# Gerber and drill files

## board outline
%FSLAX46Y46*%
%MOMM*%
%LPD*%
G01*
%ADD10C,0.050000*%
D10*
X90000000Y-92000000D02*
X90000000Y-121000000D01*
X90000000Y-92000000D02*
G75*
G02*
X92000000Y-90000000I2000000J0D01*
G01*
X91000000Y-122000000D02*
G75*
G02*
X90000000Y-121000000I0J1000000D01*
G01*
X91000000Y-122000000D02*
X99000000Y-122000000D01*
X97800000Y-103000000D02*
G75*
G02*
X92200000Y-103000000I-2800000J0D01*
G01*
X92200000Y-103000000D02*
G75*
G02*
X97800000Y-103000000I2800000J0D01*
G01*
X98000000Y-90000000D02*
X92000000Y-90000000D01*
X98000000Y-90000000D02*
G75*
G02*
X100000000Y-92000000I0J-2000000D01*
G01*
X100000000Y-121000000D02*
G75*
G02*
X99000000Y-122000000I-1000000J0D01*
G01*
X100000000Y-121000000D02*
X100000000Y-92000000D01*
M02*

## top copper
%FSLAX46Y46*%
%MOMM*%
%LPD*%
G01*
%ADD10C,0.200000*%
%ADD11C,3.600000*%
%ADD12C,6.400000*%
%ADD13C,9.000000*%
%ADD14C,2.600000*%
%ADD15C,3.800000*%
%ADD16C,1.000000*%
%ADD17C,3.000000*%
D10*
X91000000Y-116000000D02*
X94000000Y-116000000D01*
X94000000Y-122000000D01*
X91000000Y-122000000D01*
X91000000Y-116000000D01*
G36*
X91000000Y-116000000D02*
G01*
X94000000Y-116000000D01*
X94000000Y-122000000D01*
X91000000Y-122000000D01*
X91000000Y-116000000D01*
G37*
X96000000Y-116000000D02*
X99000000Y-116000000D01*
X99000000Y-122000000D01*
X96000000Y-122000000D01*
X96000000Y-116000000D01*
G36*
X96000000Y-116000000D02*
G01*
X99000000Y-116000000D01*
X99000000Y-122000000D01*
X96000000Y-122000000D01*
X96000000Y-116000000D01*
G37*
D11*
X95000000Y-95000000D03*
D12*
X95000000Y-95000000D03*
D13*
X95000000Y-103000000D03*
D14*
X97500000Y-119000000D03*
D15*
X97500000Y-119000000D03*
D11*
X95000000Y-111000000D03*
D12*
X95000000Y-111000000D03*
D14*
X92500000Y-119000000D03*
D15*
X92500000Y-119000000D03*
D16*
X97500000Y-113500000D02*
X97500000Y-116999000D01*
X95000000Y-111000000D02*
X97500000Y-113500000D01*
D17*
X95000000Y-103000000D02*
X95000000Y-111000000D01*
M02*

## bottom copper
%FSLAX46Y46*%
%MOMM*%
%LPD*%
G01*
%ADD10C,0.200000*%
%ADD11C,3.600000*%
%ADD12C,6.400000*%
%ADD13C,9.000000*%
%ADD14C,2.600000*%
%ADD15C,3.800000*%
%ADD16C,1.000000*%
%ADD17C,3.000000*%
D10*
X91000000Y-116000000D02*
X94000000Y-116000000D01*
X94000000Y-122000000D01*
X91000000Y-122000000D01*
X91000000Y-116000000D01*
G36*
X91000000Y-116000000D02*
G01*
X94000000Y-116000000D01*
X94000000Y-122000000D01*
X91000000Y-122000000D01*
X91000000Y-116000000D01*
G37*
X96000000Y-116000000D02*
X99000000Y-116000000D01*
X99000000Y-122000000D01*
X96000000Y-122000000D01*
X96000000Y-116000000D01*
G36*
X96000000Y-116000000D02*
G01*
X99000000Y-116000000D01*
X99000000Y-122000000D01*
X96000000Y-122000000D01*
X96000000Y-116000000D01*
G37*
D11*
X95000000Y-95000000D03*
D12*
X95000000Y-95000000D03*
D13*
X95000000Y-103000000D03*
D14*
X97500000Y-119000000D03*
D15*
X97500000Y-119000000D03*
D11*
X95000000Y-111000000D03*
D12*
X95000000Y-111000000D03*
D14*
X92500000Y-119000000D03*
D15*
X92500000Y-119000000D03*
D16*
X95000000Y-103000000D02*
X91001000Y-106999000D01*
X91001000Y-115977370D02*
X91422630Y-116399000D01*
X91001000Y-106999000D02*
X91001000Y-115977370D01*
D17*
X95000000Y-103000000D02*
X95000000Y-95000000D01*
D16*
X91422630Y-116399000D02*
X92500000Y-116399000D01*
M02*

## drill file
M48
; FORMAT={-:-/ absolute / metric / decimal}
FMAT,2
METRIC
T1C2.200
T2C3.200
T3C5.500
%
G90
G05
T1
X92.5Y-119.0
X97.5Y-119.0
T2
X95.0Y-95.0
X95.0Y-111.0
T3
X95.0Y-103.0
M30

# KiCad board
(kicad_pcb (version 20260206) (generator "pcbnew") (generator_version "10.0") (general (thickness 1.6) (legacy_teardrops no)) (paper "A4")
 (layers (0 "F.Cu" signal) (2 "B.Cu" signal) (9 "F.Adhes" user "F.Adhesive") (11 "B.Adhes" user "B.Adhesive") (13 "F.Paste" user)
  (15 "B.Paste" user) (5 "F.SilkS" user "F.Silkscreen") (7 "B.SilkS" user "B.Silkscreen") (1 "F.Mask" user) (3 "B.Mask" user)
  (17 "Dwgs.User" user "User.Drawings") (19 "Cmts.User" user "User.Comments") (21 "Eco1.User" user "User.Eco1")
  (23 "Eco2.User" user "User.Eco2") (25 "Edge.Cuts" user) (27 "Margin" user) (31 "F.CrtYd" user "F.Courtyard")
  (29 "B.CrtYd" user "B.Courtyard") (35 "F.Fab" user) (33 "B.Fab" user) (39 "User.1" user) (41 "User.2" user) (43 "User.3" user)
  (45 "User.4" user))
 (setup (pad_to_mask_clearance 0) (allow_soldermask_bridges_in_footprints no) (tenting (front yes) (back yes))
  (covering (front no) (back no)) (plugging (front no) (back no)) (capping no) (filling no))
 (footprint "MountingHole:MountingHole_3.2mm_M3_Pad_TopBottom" (layer "F.Cu") (at 95 95)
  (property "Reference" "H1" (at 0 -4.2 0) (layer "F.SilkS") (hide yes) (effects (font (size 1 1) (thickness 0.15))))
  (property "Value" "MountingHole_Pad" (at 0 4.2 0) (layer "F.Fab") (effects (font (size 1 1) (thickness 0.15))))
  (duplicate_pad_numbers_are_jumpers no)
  (pad "1" thru_hole circle (at 0 0) (size 3.6 3.6) (drill 3.2) (layers "*.Cu" "*.Mask") (remove_unused_layers no)
   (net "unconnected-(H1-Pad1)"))
  (pad "1" connect circle (at 0 0) (size 6.4 6.4) (layers "F.Cu" "F.Mask") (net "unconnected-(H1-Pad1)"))
  (pad "1" connect circle (at 0 0) (size 6.4 6.4) (layers "B.Cu" "B.Mask") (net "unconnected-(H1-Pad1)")))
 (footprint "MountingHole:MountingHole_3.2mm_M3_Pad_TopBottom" (layer "F.Cu") (at 95 103)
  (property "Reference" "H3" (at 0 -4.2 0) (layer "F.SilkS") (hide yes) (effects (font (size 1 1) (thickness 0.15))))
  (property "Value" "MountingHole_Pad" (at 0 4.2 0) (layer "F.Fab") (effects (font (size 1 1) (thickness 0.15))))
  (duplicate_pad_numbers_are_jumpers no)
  (pad "" np_thru_hole circle (at 0 0) (size 5.5 5.5) (drill 5.5) (layers "*.Cu" "*.Mask"))
  (pad "1" connect circle (at 0 0) (size 9 9) (layers "F.Cu" "F.Mask") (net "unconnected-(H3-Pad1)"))
  (pad "e" connect circle (at 0 0) (size 9 9) (layers "B.Cu" "B.Mask")))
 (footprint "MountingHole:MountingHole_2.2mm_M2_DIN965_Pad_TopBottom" (layer "F.Cu") (at 97.5 119)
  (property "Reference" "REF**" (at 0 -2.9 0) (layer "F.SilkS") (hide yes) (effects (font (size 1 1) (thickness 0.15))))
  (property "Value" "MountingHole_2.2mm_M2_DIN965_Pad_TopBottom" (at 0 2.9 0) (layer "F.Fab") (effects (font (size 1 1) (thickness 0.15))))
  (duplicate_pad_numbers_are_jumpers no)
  (pad "1" thru_hole circle (at 0 0) (size 2.6 2.6) (drill 2.2) (layers "*.Cu" "*.Mask") (remove_unused_layers no))
  (pad "1" connect circle (at 0 0) (size 3.8 3.8) (layers "F.Cu" "F.Mask") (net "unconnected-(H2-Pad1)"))
  (pad "1" connect circle (at 0 0) (size 3.8 3.8) (layers "B.Cu" "B.Mask") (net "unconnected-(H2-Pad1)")))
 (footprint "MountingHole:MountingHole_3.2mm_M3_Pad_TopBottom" (layer "F.Cu") (at 95 111)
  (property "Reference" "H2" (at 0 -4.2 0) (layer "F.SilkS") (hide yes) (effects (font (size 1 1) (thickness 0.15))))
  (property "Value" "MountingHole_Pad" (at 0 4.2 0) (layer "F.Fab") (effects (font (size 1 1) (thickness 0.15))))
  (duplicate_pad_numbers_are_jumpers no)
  (pad "1" thru_hole circle (at 0 0) (size 3.6 3.6) (drill 3.2) (layers "*.Cu" "*.Mask") (remove_unused_layers no)
   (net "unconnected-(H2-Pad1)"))
  (pad "1" connect circle (at 0 0) (size 6.4 6.4) (layers "F.Cu" "F.Mask") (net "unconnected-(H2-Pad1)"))
  (pad "1" connect circle (at 0 0) (size 6.4 6.4) (layers "B.Cu" "B.Mask") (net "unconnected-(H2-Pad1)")))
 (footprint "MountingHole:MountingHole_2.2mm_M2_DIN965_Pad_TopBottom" (layer "F.Cu") (at 92.5 119)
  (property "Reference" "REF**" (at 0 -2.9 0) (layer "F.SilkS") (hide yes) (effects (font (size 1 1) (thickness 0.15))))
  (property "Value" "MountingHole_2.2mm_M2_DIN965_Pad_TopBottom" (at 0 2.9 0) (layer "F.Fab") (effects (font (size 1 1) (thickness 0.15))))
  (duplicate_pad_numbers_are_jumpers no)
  (pad "1" thru_hole circle (at 0 0) (size 2.6 2.6) (drill 2.2) (layers "*.Cu" "*.Mask") (remove_unused_layers no))
  (pad "1" connect circle (at 0 0) (size 3.8 3.8) (layers "F.Cu" "F.Mask") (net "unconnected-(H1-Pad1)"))
  (pad "1" connect circle (at 0 0) (size 3.8 3.8) (layers "B.Cu" "B.Mask")))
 (gr_rect (start 91 116) (end 94 122) (stroke (width 0.2) (type solid)) (fill yes) (layers "F.Cu" "F.Mask") (net "unconnected-(H1-Pad1)"))
 (gr_rect (start 96 116) (end 99 122) (stroke (width 0.2) (type solid)) (fill yes) (layers "F.Cu" "F.Mask") (net "unconnected-(H2-Pad1)"))
 (gr_rect (start 91 116) (end 94 122) (stroke (width 0.2) (type solid)) (fill yes) (layers "B.Cu" "B.Mask") (net "unconnected-(H1-Pad1)"))
 (gr_rect (start 96 116) (end 99 122) (stroke (width 0.2) (type solid)) (fill yes) (layers "B.Cu" "B.Mask") (net "unconnected-(H2-Pad1)"))
 (gr_line (start 90 92) (end 90 121) (stroke (width 0.05) (type default)) (layer "Edge.Cuts"))
 (gr_arc (start 90 92) (mid 90.585786 90.585786) (end 92 90) (stroke (width 0.05) (type default)) (layer "Edge.Cuts"))
 (gr_arc (start 91 122) (mid 90.292893 121.707107) (end 90 121) (stroke (width 0.05) (type default)) (layer "Edge.Cuts"))
 (gr_line (start 91 122) (end 99 122) (stroke (width 0.05) (type default)) (layer "Edge.Cuts"))
 (gr_circle (center 95 103) (end 97.8 103) (stroke (width 0.05) (type solid)) (fill no) (layer "Edge.Cuts"))
 (gr_line (start 98 90) (end 92 90) (stroke (width 0.05) (type default)) (layer "Edge.Cuts"))
 (gr_arc (start 98 90) (mid 99.414214 90.585786) (end 100 92) (stroke (width 0.05) (type default)) (layer "Edge.Cuts"))
 (gr_arc (start 100 121) (mid 99.707107 121.707107) (end 99 122) (stroke (width 0.05) (type default)) (layer "Edge.Cuts"))
 (gr_line (start 100 121) (end 100 92) (stroke (width 0.05) (type default)) (layer "Edge.Cuts"))
 (segment (start 95 103) (end 91.001 106.999) (width 1) (layer "B.Cu") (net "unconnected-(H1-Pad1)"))
 (segment (start 91.001 115.97737) (end 91.42263 116.399) (width 1) (layer "B.Cu") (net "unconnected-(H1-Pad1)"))
 (segment (start 91.001 106.999) (end 91.001 115.97737) (width 1) (layer "B.Cu") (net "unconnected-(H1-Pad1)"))
 (segment (start 95 103) (end 95 95) (width 3) (layer "B.Cu") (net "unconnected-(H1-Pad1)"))
 (segment (start 91.42263 116.399) (end 92.5 116.399) (width 1) (layer "B.Cu") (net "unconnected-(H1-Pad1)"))
 (segment (start 97.5 113.5) (end 97.5 116.999) (width 1) (layer "F.Cu") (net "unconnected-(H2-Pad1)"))
 (segment (start 95 111) (end 97.5 113.5) (width 1) (layer "F.Cu") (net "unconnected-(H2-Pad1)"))
 (segment (start 95 103) (end 95 111) (width 3) (layer "F.Cu") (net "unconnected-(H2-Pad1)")))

